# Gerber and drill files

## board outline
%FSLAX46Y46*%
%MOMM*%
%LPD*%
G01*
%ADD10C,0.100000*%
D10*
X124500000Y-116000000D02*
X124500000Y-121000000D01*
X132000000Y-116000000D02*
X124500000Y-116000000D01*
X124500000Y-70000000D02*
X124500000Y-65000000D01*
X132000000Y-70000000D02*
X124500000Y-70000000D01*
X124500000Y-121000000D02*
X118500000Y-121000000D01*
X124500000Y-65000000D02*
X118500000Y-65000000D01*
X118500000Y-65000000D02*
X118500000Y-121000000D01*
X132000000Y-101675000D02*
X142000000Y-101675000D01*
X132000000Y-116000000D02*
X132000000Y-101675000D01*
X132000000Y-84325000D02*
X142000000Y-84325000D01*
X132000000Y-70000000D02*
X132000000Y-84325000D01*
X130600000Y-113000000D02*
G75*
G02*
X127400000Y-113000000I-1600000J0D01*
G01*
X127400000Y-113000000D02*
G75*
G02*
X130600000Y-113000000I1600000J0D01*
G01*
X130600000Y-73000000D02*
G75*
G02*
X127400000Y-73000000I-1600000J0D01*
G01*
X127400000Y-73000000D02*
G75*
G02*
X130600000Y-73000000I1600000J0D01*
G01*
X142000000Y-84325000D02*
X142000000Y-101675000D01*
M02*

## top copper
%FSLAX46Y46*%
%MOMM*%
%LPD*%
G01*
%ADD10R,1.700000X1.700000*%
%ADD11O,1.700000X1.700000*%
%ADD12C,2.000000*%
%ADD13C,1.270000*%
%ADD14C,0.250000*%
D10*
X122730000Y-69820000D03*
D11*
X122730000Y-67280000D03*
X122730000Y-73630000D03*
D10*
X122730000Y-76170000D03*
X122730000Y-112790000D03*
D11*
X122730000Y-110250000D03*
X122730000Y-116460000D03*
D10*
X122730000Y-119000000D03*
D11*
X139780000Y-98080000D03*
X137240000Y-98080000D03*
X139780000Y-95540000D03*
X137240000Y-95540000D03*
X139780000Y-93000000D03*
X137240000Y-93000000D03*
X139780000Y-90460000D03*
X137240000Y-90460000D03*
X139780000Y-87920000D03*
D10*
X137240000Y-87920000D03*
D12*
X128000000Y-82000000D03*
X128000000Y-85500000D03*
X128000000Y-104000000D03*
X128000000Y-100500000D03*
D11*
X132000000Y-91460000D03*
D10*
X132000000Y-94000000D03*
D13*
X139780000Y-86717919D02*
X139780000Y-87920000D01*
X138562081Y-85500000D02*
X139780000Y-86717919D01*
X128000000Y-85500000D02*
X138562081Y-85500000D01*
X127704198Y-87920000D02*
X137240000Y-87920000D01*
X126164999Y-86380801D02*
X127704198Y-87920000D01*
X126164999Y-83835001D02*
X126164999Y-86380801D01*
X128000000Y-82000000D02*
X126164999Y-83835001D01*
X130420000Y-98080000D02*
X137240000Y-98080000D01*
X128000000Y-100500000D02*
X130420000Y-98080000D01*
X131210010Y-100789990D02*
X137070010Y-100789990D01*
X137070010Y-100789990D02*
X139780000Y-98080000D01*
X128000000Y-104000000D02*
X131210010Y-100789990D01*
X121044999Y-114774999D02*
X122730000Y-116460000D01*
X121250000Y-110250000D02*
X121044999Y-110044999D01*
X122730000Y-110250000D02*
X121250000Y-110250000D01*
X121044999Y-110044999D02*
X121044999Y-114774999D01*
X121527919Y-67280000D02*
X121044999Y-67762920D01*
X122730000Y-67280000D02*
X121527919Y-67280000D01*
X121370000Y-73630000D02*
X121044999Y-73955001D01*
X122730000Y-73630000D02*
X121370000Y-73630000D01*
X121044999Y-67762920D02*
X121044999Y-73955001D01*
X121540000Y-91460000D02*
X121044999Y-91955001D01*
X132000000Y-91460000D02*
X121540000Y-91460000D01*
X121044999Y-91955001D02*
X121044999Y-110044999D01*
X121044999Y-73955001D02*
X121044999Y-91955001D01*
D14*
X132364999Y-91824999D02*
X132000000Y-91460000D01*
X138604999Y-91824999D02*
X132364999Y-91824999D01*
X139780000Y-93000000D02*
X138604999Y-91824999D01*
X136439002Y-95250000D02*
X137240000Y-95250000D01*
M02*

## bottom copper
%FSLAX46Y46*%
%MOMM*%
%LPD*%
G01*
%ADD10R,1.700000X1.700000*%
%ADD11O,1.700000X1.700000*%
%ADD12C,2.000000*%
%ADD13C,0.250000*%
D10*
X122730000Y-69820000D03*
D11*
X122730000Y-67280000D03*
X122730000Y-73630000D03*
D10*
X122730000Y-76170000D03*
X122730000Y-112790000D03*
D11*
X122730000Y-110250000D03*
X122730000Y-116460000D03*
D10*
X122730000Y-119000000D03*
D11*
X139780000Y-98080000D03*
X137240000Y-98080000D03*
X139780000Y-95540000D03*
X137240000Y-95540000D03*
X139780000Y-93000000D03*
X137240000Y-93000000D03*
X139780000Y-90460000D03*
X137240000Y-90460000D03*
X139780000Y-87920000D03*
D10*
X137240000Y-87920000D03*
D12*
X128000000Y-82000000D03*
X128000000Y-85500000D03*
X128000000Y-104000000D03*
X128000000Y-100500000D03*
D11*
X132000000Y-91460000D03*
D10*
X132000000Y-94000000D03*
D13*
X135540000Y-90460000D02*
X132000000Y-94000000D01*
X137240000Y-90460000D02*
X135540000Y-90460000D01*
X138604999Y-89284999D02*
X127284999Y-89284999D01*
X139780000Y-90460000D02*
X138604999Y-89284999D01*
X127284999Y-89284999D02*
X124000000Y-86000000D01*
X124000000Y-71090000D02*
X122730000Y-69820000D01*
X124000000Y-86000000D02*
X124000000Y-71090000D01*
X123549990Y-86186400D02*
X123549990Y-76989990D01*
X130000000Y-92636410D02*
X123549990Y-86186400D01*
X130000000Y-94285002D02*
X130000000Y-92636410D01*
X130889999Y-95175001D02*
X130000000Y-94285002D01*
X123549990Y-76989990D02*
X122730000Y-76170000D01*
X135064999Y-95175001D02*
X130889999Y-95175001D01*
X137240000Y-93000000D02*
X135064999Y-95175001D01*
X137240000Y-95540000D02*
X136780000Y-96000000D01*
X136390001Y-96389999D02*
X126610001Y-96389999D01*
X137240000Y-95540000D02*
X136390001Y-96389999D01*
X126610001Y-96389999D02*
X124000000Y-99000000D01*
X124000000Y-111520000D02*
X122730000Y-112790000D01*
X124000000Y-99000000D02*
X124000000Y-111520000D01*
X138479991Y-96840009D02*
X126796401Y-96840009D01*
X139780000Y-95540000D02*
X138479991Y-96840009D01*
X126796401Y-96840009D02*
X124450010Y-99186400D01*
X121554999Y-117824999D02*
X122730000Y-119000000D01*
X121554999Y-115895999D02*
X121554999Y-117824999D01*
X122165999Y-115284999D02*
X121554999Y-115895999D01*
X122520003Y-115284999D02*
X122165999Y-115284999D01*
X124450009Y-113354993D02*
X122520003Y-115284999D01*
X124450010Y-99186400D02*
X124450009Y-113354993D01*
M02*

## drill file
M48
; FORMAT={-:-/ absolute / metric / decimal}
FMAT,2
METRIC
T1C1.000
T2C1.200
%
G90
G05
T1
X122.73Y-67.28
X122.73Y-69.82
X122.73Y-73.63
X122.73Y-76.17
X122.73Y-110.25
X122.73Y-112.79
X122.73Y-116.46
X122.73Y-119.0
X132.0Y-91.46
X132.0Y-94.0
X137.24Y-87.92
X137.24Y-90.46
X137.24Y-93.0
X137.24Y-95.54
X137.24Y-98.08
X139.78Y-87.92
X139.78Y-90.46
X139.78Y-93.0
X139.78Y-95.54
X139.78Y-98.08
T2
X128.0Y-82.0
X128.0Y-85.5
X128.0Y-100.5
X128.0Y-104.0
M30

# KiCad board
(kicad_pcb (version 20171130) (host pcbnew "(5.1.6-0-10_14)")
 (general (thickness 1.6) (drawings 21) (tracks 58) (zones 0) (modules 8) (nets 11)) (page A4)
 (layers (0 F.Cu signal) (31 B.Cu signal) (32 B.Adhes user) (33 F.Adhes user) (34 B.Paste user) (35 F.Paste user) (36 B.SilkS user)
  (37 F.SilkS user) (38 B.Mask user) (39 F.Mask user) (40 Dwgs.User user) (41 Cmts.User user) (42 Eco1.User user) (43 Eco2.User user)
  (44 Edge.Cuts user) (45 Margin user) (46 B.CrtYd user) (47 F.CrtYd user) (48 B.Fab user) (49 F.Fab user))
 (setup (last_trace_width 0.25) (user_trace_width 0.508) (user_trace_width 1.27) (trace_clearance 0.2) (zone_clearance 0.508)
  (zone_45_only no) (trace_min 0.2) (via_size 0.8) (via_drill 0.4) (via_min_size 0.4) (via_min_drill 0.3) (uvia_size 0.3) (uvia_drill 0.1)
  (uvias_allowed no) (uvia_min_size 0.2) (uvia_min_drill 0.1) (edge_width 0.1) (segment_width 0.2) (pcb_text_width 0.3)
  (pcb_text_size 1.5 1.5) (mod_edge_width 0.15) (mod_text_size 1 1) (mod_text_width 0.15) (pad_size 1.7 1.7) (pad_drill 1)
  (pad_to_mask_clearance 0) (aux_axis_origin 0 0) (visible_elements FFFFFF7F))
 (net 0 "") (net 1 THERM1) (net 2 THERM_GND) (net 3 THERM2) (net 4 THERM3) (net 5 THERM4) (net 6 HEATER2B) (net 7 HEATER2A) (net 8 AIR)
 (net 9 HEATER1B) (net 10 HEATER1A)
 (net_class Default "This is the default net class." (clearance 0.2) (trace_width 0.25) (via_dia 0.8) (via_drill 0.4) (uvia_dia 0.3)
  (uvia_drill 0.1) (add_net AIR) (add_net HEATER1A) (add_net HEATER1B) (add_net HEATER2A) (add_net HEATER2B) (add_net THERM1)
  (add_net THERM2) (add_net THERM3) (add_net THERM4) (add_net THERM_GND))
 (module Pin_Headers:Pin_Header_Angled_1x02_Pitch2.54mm (layer F.Cu) (at 122.73 69.82 180)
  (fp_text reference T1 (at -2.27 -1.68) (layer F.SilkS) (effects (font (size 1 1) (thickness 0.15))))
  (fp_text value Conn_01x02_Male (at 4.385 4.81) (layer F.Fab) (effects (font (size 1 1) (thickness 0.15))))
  (pad 1 thru_hole rect (at 0 0 180) (size 1.7 1.7) (drill 1) (layers *.Cu *.Mask) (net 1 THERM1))
  (pad 2 thru_hole oval (at 0 2.54 180) (size 1.7 1.7) (drill 1) (layers *.Cu *.Mask) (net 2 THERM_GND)))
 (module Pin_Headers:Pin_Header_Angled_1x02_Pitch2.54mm (layer F.Cu) (at 122.73 76.17 180)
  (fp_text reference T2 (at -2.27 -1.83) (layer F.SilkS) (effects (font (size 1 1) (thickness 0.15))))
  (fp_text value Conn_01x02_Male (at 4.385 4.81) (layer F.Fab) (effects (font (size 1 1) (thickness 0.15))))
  (pad 2 thru_hole oval (at 0 2.54 180) (size 1.7 1.7) (drill 1) (layers *.Cu *.Mask) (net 2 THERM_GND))
  (pad 1 thru_hole rect (at 0 0 180) (size 1.7 1.7) (drill 1) (layers *.Cu *.Mask) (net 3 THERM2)))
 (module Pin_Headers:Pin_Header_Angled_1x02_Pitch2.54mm (layer F.Cu) (at 122.73 112.79 180)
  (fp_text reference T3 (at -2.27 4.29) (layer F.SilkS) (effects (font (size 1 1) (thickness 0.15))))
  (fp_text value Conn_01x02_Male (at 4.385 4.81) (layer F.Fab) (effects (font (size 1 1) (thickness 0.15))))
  (pad 1 thru_hole rect (at 0 0 180) (size 1.7 1.7) (drill 1) (layers *.Cu *.Mask) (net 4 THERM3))
  (pad 2 thru_hole oval (at 0 2.54 180) (size 1.7 1.7) (drill 1) (layers *.Cu *.Mask) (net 2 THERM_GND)))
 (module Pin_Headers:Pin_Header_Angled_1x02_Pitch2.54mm (layer F.Cu) (at 122.73 119 180)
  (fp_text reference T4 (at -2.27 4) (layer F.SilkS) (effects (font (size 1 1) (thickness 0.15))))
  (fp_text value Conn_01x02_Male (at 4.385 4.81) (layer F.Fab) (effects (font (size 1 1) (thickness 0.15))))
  (pad 2 thru_hole oval (at 0 2.54 180) (size 1.7 1.7) (drill 1) (layers *.Cu *.Mask) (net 2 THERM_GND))
  (pad 1 thru_hole rect (at 0 0 180) (size 1.7 1.7) (drill 1) (layers *.Cu *.Mask) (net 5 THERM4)))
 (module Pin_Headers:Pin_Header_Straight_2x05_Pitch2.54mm (layer F.Cu) (at 137.24 87.92)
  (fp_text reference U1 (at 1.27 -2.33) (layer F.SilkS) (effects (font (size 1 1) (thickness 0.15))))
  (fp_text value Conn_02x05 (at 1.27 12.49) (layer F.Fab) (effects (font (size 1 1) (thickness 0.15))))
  (pad 10 thru_hole oval (at 2.54 10.16) (size 1.7 1.7) (drill 1) (layers *.Cu *.Mask) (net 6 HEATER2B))
  (pad 9 thru_hole oval (at 0 10.16) (size 1.7 1.7) (drill 1) (layers *.Cu *.Mask) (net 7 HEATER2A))
  (pad 8 thru_hole oval (at 2.54 7.62) (size 1.7 1.7) (drill 1) (layers *.Cu *.Mask) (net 5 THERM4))
  (pad 7 thru_hole oval (at 0 7.62) (size 1.7 1.7) (drill 1) (layers *.Cu *.Mask) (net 4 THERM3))
  (pad 6 thru_hole oval (at 2.54 5.08) (size 1.7 1.7) (drill 1) (layers *.Cu *.Mask) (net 2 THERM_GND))
  (pad 5 thru_hole oval (at 0 5.08) (size 1.7 1.7) (drill 1) (layers *.Cu *.Mask) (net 3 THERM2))
  (pad 4 thru_hole oval (at 2.54 2.54) (size 1.7 1.7) (drill 1) (layers *.Cu *.Mask) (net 1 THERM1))
  (pad 3 thru_hole oval (at 0 2.54) (size 1.7 1.7) (drill 1) (layers *.Cu *.Mask) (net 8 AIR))
  (pad 2 thru_hole oval (at 2.54 0) (size 1.7 1.7) (drill 1) (layers *.Cu *.Mask) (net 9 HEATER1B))
  (pad 1 thru_hole rect (at 0 0) (size 1.7 1.7) (drill 1) (layers *.Cu *.Mask) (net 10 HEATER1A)))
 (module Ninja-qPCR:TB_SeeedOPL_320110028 (layer F.Cu) (at 128 82 270)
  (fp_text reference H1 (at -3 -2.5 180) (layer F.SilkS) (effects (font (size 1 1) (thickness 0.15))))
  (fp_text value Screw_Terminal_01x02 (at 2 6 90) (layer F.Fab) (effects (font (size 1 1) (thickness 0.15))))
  (pad 1 thru_hole circle (at 0 0 270) (size 2 2) (drill 1.2) (layers *.Cu *.Mask) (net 10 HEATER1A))
  (pad 2 thru_hole circle (at 3.5 0 270) (size 2 2) (drill 1.2) (layers *.Cu *.Mask) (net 9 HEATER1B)))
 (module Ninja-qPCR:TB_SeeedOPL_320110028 (layer F.Cu) (at 128 100.5 270)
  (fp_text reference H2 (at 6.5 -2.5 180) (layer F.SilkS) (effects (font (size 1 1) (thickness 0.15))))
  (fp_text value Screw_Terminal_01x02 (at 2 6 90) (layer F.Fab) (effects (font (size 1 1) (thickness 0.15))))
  (pad 2 thru_hole circle (at 3.5 0 270) (size 2 2) (drill 1.2) (layers *.Cu *.Mask) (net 6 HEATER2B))
  (pad 1 thru_hole circle (at 0 0 270) (size 2 2) (drill 1.2) (layers *.Cu *.Mask) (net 7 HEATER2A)))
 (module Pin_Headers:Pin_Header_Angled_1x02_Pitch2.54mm (layer F.Cu) (at 132 94 180)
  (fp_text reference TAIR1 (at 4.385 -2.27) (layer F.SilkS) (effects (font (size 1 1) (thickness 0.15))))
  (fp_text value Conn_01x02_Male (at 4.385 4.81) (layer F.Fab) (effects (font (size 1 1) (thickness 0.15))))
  (pad 2 thru_hole oval (at 0 2.54 180) (size 1.7 1.7) (drill 1) (layers *.Cu *.Mask) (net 2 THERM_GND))
  (pad 1 thru_hole rect (at 0 0 180) (size 1.7 1.7) (drill 1) (layers *.Cu *.Mask) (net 8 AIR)))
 (gr_line (start 124.5 116) (end 124.5 121) (layer Edge.Cuts) (width 0.1))
 (gr_line (start 132 116) (end 124.5 116) (layer Edge.Cuts) (width 0.1))
 (gr_line (start 124.5 70) (end 124.5 65) (layer Edge.Cuts) (width 0.1))
 (gr_line (start 132 70) (end 124.5 70) (layer Edge.Cuts) (width 0.1))
 (gr_line (start 124.5 121) (end 118.5 121) (layer Edge.Cuts) (width 0.1))
 (gr_line (start 124.5 65) (end 118.5 65) (layer Edge.Cuts) (width 0.1))
 (gr_line (start 118.5 65) (end 118.5 121) (layer Edge.Cuts) (width 0.1))
 (gr_line (start 132 101.675) (end 142 101.675) (layer Edge.Cuts) (width 0.1))
 (gr_line (start 132 116) (end 132 101.675) (layer Edge.Cuts) (width 0.1))
 (gr_line (start 132 84.325) (end 142 84.325) (layer Edge.Cuts) (width 0.1))
 (gr_line (start 132 70) (end 132 84.325) (layer Edge.Cuts) (width 0.1))
 (gr_circle (center 129 113) (end 130.6 113) (layer Edge.Cuts) (width 0.1))
 (gr_circle (center 129 73) (end 130.6 73) (layer Edge.Cuts) (width 0.1))
 (gr_line (start 142 84.325) (end 142 101.675) (layer Edge.Cuts) (width 0.1))
 (segment (start 139.78 86.717919) (end 139.78 87.92) (width 1.27) (layer F.Cu) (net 9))
 (segment (start 138.562081 85.5) (end 139.78 86.717919) (width 1.27) (layer F.Cu) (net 9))
 (segment (start 128 85.5) (end 138.562081 85.5) (width 1.27) (layer F.Cu) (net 9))
 (segment (start 127.704198 87.92) (end 137.24 87.92) (width 1.27) (layer F.Cu) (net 10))
 (segment (start 126.164999 86.380801) (end 127.704198 87.92) (width 1.27) (layer F.Cu) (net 10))
 (segment (start 126.164999 83.835001) (end 126.164999 86.380801) (width 1.27) (layer F.Cu) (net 10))
 (segment (start 128 82) (end 126.164999 83.835001) (width 1.27) (layer F.Cu) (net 10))
 (segment (start 130.42 98.08) (end 137.24 98.08) (width 1.27) (layer F.Cu) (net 7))
 (segment (start 128 100.5) (end 130.42 98.08) (width 1.27) (layer F.Cu) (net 7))
 (segment (start 131.21001 100.78999) (end 137.07001 100.78999) (width 1.27) (layer F.Cu) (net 6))
 (segment (start 137.07001 100.78999) (end 139.78 98.08) (width 1.27) (layer F.Cu) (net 6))
 (segment (start 128 104) (end 131.21001 100.78999) (width 1.27) (layer F.Cu) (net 6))
 (segment (start 121.044999 114.774999) (end 122.73 116.46) (width 1.27) (layer F.Cu) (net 2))
 (segment (start 121.25 110.25) (end 121.044999 110.044999) (width 1.27) (layer F.Cu) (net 2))
 (segment (start 122.73 110.25) (end 121.25 110.25) (width 1.27) (layer F.Cu) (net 2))
 (segment (start 121.044999 110.044999) (end 121.044999 114.774999) (width 1.27) (layer F.Cu) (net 2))
 (segment (start 121.527919 67.28) (end 121.044999 67.76292) (width 1.27) (layer F.Cu) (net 2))
 (segment (start 122.73 67.28) (end 121.527919 67.28) (width 1.27) (layer F.Cu) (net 2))
 (segment (start 121.37 73.63) (end 121.044999 73.955001) (width 1.27) (layer F.Cu) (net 2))
 (segment (start 122.73 73.63) (end 121.37 73.63) (width 1.27) (layer F.Cu) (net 2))
 (segment (start 121.044999 67.76292) (end 121.044999 73.955001) (width 1.27) (layer F.Cu) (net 2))
 (segment (start 121.54 91.46) (end 121.044999 91.955001) (width 1.27) (layer F.Cu) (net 2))
 (segment (start 132 91.46) (end 121.54 91.46) (width 1.27) (layer F.Cu) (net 2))
 (segment (start 121.044999 91.955001) (end 121.044999 110.044999) (width 1.27) (layer F.Cu) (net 2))
 (segment (start 121.044999 73.955001) (end 121.044999 91.955001) (width 1.27) (layer F.Cu) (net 2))
 (segment (start 132.364999 91.824999) (end 132 91.46) (width 0.25) (layer F.Cu) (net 2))
 (segment (start 138.604999 91.824999) (end 132.364999 91.824999) (width 0.25) (layer F.Cu) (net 2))
 (segment (start 139.78 93) (end 138.604999 91.824999) (width 0.25) (layer F.Cu) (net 2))
 (segment (start 135.54 90.46) (end 132 94) (width 0.25) (layer B.Cu) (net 8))
 (segment (start 137.24 90.46) (end 135.54 90.46) (width 0.25) (layer B.Cu) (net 8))
 (segment (start 138.604999 89.284999) (end 127.284999 89.284999) (width 0.25) (layer B.Cu) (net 1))
 (segment (start 139.78 90.46) (end 138.604999 89.284999) (width 0.25) (layer B.Cu) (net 1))
 (segment (start 127.284999 89.284999) (end 124 86) (width 0.25) (layer B.Cu) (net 1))
 (segment (start 124 71.09) (end 122.73 69.82) (width 0.25) (layer B.Cu) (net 1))
 (segment (start 124 86) (end 124 71.09) (width 0.25) (layer B.Cu) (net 1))
 (segment (start 123.54999 86.1864) (end 123.54999 76.98999) (width 0.25) (layer B.Cu) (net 3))
 (segment (start 130 92.63641) (end 123.54999 86.1864) (width 0.25) (layer B.Cu) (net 3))
 (segment (start 130 94.285002) (end 130 92.63641) (width 0.25) (layer B.Cu) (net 3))
 (segment (start 130.889999 95.175001) (end 130 94.285002) (width 0.25) (layer B.Cu) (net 3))
 (segment (start 123.54999 76.98999) (end 122.73 76.17) (width 0.25) (layer B.Cu) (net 3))
 (segment (start 135.064999 95.175001) (end 130.889999 95.175001) (width 0.25) (layer B.Cu) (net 3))
 (segment (start 137.24 93) (end 135.064999 95.175001) (width 0.25) (layer B.Cu) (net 3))
 (segment (start 136.439002 95.25) (end 137.24 95.25) (width 0.25) (layer F.Cu) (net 4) (status 20))
 (segment (start 137.24 95.54) (end 136.78 96) (width 0.25) (layer B.Cu) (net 4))
 (segment (start 136.390001 96.389999) (end 126.610001 96.389999) (width 0.25) (layer B.Cu) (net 4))
 (segment (start 137.24 95.54) (end 136.390001 96.389999) (width 0.25) (layer B.Cu) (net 4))
 (segment (start 126.610001 96.389999) (end 124 99) (width 0.25) (layer B.Cu) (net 4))
 (segment (start 124 111.52) (end 122.73 112.79) (width 0.25) (layer B.Cu) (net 4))
 (segment (start 124 99) (end 124 111.52) (width 0.25) (layer B.Cu) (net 4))
 (segment (start 138.479991 96.840009) (end 126.796401 96.840009) (width 0.25) (layer B.Cu) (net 5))
 (segment (start 139.78 95.54) (end 138.479991 96.840009) (width 0.25) (layer B.Cu) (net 5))
 (segment (start 126.796401 96.840009) (end 124.45001 99.1864) (width 0.25) (layer B.Cu) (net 5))
 (segment (start 121.554999 117.824999) (end 122.73 119) (width 0.25) (layer B.Cu) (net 5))
 (segment (start 121.554999 115.895999) (end 121.554999 117.824999) (width 0.25) (layer B.Cu) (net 5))
 (segment (start 122.165999 115.284999) (end 121.554999 115.895999) (width 0.25) (layer B.Cu) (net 5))
 (segment (start 122.520003 115.284999) (end 122.165999 115.284999) (width 0.25) (layer B.Cu) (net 5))
 (segment (start 124.450009 113.354993) (end 122.520003 115.284999) (width 0.25) (layer B.Cu) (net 5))
 (segment (start 124.45001 99.1864) (end 124.450009 113.354993) (width 0.25) (layer B.Cu) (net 5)))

